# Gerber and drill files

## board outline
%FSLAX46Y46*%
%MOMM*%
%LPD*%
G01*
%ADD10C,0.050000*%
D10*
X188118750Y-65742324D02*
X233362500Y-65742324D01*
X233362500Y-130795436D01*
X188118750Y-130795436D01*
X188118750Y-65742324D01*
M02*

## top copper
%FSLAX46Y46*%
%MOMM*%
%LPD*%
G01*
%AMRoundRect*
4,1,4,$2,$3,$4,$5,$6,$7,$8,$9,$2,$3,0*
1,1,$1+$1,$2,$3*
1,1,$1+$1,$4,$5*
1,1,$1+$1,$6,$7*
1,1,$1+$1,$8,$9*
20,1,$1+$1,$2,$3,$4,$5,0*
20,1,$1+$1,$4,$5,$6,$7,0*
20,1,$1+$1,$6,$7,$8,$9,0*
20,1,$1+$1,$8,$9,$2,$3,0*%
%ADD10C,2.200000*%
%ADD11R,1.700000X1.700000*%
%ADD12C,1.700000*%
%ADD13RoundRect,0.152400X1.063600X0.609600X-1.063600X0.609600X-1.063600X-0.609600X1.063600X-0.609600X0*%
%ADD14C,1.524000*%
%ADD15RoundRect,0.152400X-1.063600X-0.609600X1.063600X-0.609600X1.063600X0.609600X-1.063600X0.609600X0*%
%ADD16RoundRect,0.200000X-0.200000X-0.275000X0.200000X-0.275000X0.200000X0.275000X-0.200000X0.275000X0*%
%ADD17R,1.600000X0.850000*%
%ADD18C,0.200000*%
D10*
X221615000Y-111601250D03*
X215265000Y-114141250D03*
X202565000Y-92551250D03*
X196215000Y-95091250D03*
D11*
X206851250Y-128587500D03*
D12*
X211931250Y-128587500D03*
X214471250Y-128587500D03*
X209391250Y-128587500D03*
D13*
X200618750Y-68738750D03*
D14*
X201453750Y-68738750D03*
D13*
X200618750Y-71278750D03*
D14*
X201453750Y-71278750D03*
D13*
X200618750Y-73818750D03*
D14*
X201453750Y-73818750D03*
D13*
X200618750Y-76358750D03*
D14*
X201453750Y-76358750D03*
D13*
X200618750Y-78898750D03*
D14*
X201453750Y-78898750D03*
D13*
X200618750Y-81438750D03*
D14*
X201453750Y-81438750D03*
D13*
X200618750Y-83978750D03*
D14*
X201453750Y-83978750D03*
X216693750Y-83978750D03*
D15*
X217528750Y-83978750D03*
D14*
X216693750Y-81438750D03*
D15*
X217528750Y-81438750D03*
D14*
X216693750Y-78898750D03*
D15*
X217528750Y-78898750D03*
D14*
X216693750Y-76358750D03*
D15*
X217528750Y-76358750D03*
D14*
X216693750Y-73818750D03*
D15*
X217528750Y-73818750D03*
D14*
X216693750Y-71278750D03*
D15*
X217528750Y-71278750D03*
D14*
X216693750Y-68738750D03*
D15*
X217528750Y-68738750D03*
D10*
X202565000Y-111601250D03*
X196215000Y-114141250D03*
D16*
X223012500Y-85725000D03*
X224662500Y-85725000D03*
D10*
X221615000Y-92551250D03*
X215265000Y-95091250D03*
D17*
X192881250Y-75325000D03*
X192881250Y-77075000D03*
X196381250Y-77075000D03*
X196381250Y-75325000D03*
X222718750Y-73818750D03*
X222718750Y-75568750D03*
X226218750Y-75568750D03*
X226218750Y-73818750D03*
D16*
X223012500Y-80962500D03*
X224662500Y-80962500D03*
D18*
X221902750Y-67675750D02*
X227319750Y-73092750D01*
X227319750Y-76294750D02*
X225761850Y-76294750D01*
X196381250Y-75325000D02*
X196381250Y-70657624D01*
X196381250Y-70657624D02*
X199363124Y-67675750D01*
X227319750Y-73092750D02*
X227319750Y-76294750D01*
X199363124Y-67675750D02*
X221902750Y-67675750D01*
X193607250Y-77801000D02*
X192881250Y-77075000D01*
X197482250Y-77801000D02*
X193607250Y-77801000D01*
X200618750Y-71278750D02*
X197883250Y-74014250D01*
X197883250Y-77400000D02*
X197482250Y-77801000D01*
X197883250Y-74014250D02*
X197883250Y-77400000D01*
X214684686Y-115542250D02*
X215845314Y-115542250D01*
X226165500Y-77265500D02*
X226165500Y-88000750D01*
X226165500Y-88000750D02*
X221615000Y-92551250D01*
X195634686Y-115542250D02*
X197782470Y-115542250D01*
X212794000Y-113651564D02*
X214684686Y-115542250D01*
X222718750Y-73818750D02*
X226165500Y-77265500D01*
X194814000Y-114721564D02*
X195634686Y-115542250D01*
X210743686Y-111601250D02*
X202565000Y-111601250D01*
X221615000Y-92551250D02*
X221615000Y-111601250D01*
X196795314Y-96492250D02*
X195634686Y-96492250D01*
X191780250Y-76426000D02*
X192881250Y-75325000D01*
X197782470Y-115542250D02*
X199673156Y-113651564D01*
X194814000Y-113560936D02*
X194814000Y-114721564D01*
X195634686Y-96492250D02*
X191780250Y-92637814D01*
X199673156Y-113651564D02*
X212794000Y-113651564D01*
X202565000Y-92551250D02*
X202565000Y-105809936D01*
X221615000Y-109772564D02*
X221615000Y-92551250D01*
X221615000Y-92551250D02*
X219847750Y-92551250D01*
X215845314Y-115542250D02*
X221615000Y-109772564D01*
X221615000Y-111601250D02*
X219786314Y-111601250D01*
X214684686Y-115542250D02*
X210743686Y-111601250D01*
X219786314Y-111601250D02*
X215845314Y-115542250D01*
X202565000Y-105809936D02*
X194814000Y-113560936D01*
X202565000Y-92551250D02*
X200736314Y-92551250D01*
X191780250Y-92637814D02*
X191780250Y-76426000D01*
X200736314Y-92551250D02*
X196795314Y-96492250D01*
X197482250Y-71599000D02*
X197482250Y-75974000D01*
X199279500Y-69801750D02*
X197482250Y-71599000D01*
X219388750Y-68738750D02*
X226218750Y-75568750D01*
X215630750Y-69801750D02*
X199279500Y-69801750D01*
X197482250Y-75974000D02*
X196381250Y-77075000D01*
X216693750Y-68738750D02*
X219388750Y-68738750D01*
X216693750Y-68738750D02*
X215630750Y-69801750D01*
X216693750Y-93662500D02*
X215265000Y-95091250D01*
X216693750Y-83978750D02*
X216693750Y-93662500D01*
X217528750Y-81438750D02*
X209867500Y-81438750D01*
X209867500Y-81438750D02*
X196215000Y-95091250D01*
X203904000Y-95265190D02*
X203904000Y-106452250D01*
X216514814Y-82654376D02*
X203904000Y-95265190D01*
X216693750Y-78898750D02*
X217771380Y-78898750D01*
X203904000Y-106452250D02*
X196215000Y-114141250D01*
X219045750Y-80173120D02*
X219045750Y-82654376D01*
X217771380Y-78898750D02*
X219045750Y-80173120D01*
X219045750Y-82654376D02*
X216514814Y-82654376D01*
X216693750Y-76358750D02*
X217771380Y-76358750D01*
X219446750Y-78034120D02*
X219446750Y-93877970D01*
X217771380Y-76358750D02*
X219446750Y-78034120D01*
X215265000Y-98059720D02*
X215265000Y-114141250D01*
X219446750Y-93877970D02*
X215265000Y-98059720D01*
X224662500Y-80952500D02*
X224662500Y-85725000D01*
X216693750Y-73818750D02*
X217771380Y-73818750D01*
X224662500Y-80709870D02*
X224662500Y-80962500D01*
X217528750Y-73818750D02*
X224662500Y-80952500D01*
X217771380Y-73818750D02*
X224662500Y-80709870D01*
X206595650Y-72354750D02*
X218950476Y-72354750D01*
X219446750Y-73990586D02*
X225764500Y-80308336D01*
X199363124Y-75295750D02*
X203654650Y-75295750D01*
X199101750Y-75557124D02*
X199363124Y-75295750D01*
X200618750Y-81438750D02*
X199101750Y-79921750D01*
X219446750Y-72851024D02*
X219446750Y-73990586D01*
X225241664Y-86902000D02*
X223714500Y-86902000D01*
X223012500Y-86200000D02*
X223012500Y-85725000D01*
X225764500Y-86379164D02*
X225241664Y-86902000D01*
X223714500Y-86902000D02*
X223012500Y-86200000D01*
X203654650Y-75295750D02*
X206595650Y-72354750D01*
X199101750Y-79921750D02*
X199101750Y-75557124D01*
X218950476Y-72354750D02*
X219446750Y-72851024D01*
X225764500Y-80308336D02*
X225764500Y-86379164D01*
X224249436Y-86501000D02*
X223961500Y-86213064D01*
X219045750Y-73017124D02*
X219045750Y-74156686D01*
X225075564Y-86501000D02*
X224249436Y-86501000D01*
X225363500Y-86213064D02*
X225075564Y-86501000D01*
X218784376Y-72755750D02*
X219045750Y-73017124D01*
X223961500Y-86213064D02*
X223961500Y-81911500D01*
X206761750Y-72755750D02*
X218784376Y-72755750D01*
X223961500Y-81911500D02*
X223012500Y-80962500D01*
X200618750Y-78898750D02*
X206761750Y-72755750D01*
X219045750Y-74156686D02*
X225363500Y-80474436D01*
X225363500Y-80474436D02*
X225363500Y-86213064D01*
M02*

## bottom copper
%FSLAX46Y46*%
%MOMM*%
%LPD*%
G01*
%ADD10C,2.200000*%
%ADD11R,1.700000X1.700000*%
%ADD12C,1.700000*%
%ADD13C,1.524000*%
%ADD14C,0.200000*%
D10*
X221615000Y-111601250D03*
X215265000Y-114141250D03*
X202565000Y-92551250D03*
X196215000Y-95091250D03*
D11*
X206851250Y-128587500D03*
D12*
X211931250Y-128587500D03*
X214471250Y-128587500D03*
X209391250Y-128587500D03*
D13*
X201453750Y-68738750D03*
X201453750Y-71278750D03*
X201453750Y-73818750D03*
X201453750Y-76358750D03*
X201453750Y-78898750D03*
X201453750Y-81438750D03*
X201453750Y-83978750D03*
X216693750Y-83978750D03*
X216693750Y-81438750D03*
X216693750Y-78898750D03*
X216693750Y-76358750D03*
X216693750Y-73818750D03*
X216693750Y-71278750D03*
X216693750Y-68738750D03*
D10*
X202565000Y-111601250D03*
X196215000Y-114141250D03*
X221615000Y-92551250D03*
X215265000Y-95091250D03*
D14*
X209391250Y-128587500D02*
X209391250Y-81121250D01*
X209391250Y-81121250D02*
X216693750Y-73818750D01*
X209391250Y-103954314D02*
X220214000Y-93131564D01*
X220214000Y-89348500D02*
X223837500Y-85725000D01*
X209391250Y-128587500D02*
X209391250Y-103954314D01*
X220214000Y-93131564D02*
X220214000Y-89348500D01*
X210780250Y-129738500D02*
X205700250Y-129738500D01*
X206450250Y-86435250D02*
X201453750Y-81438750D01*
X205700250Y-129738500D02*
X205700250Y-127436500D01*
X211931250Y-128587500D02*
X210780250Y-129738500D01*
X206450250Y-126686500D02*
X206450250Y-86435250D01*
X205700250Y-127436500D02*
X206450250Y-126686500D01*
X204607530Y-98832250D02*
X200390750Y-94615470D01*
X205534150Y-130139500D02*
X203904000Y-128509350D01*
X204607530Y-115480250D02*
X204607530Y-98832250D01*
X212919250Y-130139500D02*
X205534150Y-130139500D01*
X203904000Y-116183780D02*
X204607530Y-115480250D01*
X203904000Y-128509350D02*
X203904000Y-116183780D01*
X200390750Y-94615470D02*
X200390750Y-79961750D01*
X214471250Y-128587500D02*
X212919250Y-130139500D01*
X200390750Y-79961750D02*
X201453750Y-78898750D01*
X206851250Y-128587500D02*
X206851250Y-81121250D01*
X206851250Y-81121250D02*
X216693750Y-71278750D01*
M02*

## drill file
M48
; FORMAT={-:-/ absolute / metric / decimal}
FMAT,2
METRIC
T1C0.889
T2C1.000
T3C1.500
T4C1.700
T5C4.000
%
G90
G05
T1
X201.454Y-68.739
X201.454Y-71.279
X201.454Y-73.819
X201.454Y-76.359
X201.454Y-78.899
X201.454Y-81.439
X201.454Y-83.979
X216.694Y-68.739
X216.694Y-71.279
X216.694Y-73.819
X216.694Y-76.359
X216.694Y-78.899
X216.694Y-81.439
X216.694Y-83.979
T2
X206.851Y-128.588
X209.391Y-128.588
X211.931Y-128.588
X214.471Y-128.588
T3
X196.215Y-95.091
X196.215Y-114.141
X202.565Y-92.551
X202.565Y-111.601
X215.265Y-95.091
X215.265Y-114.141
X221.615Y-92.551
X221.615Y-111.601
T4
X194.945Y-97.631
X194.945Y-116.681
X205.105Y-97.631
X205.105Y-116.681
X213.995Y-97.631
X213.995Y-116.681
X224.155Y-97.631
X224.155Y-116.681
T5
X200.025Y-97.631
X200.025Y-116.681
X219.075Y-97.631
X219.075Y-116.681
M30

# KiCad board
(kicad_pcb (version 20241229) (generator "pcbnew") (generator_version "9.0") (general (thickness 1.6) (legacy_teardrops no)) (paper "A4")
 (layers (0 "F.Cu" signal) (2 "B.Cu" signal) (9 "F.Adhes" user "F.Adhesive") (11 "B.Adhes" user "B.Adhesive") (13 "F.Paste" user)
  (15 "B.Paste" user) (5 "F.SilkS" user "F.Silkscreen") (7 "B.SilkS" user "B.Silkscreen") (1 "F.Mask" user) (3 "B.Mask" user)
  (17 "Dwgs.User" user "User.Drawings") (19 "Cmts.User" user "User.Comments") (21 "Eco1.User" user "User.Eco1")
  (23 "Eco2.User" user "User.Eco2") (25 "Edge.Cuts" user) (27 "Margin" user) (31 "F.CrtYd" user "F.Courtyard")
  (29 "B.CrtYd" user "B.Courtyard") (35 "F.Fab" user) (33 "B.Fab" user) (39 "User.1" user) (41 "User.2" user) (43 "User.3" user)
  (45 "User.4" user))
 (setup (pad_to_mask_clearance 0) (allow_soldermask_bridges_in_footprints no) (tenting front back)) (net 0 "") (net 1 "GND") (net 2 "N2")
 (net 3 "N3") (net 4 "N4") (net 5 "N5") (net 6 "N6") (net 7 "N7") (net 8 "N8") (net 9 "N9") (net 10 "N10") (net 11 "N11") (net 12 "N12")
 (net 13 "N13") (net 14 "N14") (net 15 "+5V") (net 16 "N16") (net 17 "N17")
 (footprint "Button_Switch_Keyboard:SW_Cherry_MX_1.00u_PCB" (layer "F.Cu") (at 221.615 111.60125)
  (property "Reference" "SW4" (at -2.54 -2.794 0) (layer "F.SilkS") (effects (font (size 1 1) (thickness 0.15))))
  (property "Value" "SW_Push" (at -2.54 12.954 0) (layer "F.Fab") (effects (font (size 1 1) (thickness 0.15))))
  (pad "" np_thru_hole circle (at -7.62 5.08) (size 1.7 1.7) (drill 1.7) (layers "*.Cu" "*.Mask"))
  (pad "" np_thru_hole circle (at -2.54 5.08) (size 4 4) (drill 4) (layers "*.Cu" "*.Mask"))
  (pad "" np_thru_hole circle (at 2.54 5.08) (size 1.7 1.7) (drill 1.7) (layers "*.Cu" "*.Mask"))
  (pad "1" thru_hole circle (at 0 0) (size 2.2 2.2) (drill 1.5) (layers "*.Cu" "*.Mask") (remove_unused_layers no) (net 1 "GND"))
  (pad "2" thru_hole circle (at -6.35 2.54) (size 2.2 2.2) (drill 1.5) (layers "*.Cu" "*.Mask") (remove_unused_layers no) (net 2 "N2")))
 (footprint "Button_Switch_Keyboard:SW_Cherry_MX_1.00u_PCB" (layer "F.Cu") (at 202.565 92.55125)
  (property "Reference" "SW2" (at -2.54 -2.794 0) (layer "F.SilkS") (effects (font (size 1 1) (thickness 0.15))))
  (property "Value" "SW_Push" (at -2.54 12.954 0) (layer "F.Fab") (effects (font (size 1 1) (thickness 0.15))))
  (pad "" np_thru_hole circle (at -7.62 5.08) (size 1.7 1.7) (drill 1.7) (layers "*.Cu" "*.Mask"))
  (pad "" np_thru_hole circle (at -2.54 5.08) (size 4 4) (drill 4) (layers "*.Cu" "*.Mask"))
  (pad "" np_thru_hole circle (at 2.54 5.08) (size 1.7 1.7) (drill 1.7) (layers "*.Cu" "*.Mask"))
  (pad "1" thru_hole circle (at 0 0) (size 2.2 2.2) (drill 1.5) (layers "*.Cu" "*.Mask") (remove_unused_layers no) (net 1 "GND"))
  (pad "2" thru_hole circle (at -6.35 2.54) (size 2.2 2.2) (drill 1.5) (layers "*.Cu" "*.Mask") (remove_unused_layers no) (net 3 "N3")))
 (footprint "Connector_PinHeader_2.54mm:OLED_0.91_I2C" (layer "F.Cu") (at 206.85125 128.5875 90)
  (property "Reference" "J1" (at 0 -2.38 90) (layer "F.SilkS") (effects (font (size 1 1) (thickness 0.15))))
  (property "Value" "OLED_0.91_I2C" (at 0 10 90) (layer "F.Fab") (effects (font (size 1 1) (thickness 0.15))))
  (pad "GND" thru_hole rect (at 0 0 90) (size 1.7 1.7) (drill 1) (layers "*.Cu" "*.Mask") (remove_unused_layers no) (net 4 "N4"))
  (pad "SCL" thru_hole circle (at 0 5.08 90) (size 1.7 1.7) (drill 1) (layers "*.Cu" "*.Mask") (remove_unused_layers no) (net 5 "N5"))
  (pad "SDA" thru_hole circle (at 0 7.62 90) (size 1.7 1.7) (drill 1) (layers "*.Cu" "*.Mask") (remove_unused_layers no) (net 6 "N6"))
  (pad "VCC" thru_hole circle (at 0 2.54 90) (size 1.7 1.7) (drill 1) (layers "*.Cu" "*.Mask") (remove_unused_layers no) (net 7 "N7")))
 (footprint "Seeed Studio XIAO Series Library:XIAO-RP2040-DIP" (layer "F.Cu") (at 209.07375 76.35875)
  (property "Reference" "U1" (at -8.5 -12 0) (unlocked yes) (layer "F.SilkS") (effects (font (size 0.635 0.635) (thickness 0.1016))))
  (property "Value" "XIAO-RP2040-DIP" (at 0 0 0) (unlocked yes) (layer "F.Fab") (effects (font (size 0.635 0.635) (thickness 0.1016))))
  (pad "1" smd roundrect (at -8.455 -7.62 180) (size 2.432 1.524) (layers "F.Cu" "F.Mask") (roundrect_rratio 0.1) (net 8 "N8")
   (thermal_bridge_angle 45))
  (pad "1" thru_hole circle (at -7.62 -7.62 180) (size 1.524 1.524) (drill 0.889) (layers "*.Cu" "*.Mask") (remove_unused_layers no)
   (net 8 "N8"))
  (pad "2" smd roundrect (at -8.455 -5.08 180) (size 2.432 1.524) (layers "F.Cu" "F.Mask") (roundrect_rratio 0.1) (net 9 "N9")
   (thermal_bridge_angle 45))
  (pad "2" thru_hole circle (at -7.62 -5.08 180) (size 1.524 1.524) (drill 0.889) (layers "*.Cu" "*.Mask") (remove_unused_layers no)
   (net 9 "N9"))
  (pad "3" smd roundrect (at -8.455 -2.54 180) (size 2.432 1.524) (layers "F.Cu" "F.Mask") (roundrect_rratio 0.1) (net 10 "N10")
   (thermal_bridge_angle 45))
  (pad "3" thru_hole circle (at -7.62 -2.54 180) (size 1.524 1.524) (drill 0.889) (layers "*.Cu" "*.Mask") (remove_unused_layers no)
   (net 10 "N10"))
  (pad "4" smd roundrect (at -8.455 0 180) (size 2.432 1.524) (layers "F.Cu" "F.Mask") (roundrect_rratio 0.1) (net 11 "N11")
   (thermal_bridge_angle 45))
  (pad "4" thru_hole circle (at -7.62 0 180) (size 1.524 1.524) (drill 0.889) (layers "*.Cu" "*.Mask") (remove_unused_layers no)
   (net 11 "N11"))
  (pad "5" smd roundrect (at -8.455 2.54 180) (size 2.432 1.524) (layers "F.Cu" "F.Mask") (roundrect_rratio 0.1) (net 6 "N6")
   (thermal_bridge_angle 45))
  (pad "5" thru_hole circle (at -7.62 2.54 180) (size 1.524 1.524) (drill 0.889) (layers "*.Cu" "*.Mask") (remove_unused_layers no)
   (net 6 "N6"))
  (pad "6" smd roundrect (at -8.455 5.08 180) (size 2.432 1.524) (layers "F.Cu" "F.Mask") (roundrect_rratio 0.1) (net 5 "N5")
   (thermal_bridge_angle 45))
  (pad "6" thru_hole circle (at -7.62 5.08 180) (size 1.524 1.524) (drill 0.889) (layers "*.Cu" "*.Mask") (remove_unused_layers no)
   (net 5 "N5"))
  (pad "7" smd roundrect (at -8.455 7.62 180) (size 2.432 1.524) (layers "F.Cu" "F.Mask") (roundrect_rratio 0.1) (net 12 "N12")
   (thermal_bridge_angle 45))
  (pad "7" thru_hole circle (at -7.62 7.62 180) (size 1.524 1.524) (drill 0.889) (layers "*.Cu" "*.Mask") (remove_unused_layers no)
   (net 12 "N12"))
  (pad "8" thru_hole circle (at 7.62 7.62) (size 1.524 1.524) (drill 0.889) (layers "*.Cu" "*.Mask") (remove_unused_layers no)
   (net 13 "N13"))
  (pad "8" smd roundrect (at 8.455 7.62) (size 2.432 1.524) (layers "F.Cu" "F.Mask") (roundrect_rratio 0.1) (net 13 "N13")
   (thermal_bridge_angle 45))
  (pad "9" thru_hole circle (at 7.62 5.08) (size 1.524 1.524) (drill 0.889) (layers "*.Cu" "*.Mask") (remove_unused_layers no) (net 3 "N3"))
  (pad "9" smd roundrect (at 8.455 5.08) (size 2.432 1.524) (layers "F.Cu" "F.Mask") (roundrect_rratio 0.1) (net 3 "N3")
   (thermal_bridge_angle 45))
  (pad "10" thru_hole circle (at 7.62 2.54) (size 1.524 1.524) (drill 0.889) (layers "*.Cu" "*.Mask") (remove_unused_layers no)
   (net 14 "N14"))
  (pad "10" smd roundrect (at 8.455 2.54) (size 2.432 1.524) (layers "F.Cu" "F.Mask") (roundrect_rratio 0.1) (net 14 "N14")
   (thermal_bridge_angle 45))
  (pad "11" thru_hole circle (at 7.62 0) (size 1.524 1.524) (drill 0.889) (layers "*.Cu" "*.Mask") (remove_unused_layers no) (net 2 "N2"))
  (pad "11" smd roundrect (at 8.455 0) (size 2.432 1.524) (layers "F.Cu" "F.Mask") (roundrect_rratio 0.1) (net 2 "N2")
   (thermal_bridge_angle 45))
  (pad "12" thru_hole circle (at 7.62 -2.54) (size 1.524 1.524) (drill 0.889) (layers "*.Cu" "*.Mask") (remove_unused_layers no)
   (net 7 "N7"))
  (pad "12" smd roundrect (at 8.455 -2.54) (size 2.432 1.524) (layers "F.Cu" "F.Mask") (roundrect_rratio 0.1) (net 7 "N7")
   (thermal_bridge_angle 45))
  (pad "13" thru_hole circle (at 7.62 -5.08) (size 1.524 1.524) (drill 0.889) (layers "*.Cu" "*.Mask") (remove_unused_layers no)
   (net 4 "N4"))
  (pad "13" smd roundrect (at 8.455 -5.08) (size 2.432 1.524) (layers "F.Cu" "F.Mask") (roundrect_rratio 0.1) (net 4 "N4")
   (thermal_bridge_angle 45))
  (pad "14" thru_hole circle (at 7.62 -7.62) (size 1.524 1.524) (drill 0.889) (layers "*.Cu" "*.Mask") (remove_unused_layers no)
   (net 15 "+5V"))
  (pad "14" smd roundrect (at 8.455 -7.62) (size 2.432 1.524) (layers "F.Cu" "F.Mask") (roundrect_rratio 0.1) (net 15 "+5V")
   (thermal_bridge_angle 45)))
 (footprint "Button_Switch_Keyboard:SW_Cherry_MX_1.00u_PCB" (layer "F.Cu") (at 202.565 111.60125)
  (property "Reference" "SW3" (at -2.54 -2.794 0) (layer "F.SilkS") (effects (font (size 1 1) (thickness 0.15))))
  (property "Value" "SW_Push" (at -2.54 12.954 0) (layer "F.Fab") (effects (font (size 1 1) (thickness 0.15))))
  (pad "" np_thru_hole circle (at -7.62 5.08) (size 1.7 1.7) (drill 1.7) (layers "*.Cu" "*.Mask"))
  (pad "" np_thru_hole circle (at -2.54 5.08) (size 4 4) (drill 4) (layers "*.Cu" "*.Mask"))
  (pad "" np_thru_hole circle (at 2.54 5.08) (size 1.7 1.7) (drill 1.7) (layers "*.Cu" "*.Mask"))
  (pad "1" thru_hole circle (at 0 0) (size 2.2 2.2) (drill 1.5) (layers "*.Cu" "*.Mask") (remove_unused_layers no) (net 1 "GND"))
  (pad "2" thru_hole circle (at -6.35 2.54) (size 2.2 2.2) (drill 1.5) (layers "*.Cu" "*.Mask") (remove_unused_layers no) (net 14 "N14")))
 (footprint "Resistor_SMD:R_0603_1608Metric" (layer "F.Cu") (at 223.8375 85.725)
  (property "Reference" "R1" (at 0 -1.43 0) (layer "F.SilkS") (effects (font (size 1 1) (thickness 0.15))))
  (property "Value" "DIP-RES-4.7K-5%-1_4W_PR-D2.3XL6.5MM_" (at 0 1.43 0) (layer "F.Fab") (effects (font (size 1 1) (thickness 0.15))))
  (pad "1" smd roundrect (at -0.825 0) (size 0.8 0.95) (layers "F.Cu" "F.Mask" "F.Paste") (roundrect_rratio 0.25) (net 5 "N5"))
  (pad "2" smd roundrect (at 0.825 0) (size 0.8 0.95) (layers "F.Cu" "F.Mask" "F.Paste") (roundrect_rratio 0.25) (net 7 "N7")))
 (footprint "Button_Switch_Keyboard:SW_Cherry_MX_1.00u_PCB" (layer "F.Cu") (at 221.615 92.55125)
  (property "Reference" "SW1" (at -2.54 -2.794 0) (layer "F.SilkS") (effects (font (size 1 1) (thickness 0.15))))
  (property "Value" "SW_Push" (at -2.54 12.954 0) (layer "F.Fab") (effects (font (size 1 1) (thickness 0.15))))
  (pad "" np_thru_hole circle (at -7.62 5.08) (size 1.7 1.7) (drill 1.7) (layers "*.Cu" "*.Mask"))
  (pad "" np_thru_hole circle (at -2.54 5.08) (size 4 4) (drill 4) (layers "*.Cu" "*.Mask"))
  (pad "" np_thru_hole circle (at 2.54 5.08) (size 1.7 1.7) (drill 1.7) (layers "*.Cu" "*.Mask"))
  (pad "1" thru_hole circle (at 0 0) (size 2.2 2.2) (drill 1.5) (layers "*.Cu" "*.Mask") (remove_unused_layers no) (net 1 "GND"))
  (pad "2" thru_hole circle (at -6.35 2.54) (size 2.2 2.2) (drill 1.5) (layers "*.Cu" "*.Mask") (remove_unused_layers no) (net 13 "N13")))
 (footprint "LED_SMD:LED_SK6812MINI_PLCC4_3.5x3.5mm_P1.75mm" (layer "F.Cu") (at 194.63125 76.2)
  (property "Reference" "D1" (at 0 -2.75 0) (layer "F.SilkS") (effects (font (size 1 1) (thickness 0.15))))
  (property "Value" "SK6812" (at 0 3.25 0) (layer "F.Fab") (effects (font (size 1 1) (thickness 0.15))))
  (pad "1" smd rect (at -1.75 -0.875) (size 1.6 0.85) (layers "F.Cu" "F.Mask" "F.Paste") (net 1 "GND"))
  (pad "2" smd rect (at -1.75 0.875) (size 1.6 0.85) (layers "F.Cu" "F.Mask" "F.Paste") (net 9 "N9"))
  (pad "3" smd rect (at 1.75 0.875) (size 1.6 0.85) (layers "F.Cu" "F.Mask" "F.Paste") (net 15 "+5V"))
  (pad "4" smd rect (at 1.75 -0.875) (size 1.6 0.85) (layers "F.Cu" "F.Mask" "F.Paste") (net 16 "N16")))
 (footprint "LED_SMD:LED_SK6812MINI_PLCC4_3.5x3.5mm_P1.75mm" (layer "F.Cu") (at 224.46875 74.69375)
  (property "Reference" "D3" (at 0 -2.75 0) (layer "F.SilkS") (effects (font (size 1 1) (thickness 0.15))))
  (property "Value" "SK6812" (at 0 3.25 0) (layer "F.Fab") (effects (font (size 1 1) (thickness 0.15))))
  (pad "1" smd rect (at -1.75 -0.875) (size 1.6 0.85) (layers "F.Cu" "F.Mask" "F.Paste") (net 1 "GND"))
  (pad "2" smd rect (at -1.75 0.875) (size 1.6 0.85) (layers "F.Cu" "F.Mask" "F.Paste") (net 16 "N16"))
  (pad "3" smd rect (at 1.75 0.875) (size 1.6 0.85) (layers "F.Cu" "F.Mask" "F.Paste") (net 15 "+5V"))
  (pad "4" smd rect (at 1.75 -0.875) (size 1.6 0.85) (layers "F.Cu" "F.Mask" "F.Paste") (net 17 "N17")))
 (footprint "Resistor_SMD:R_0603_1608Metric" (layer "F.Cu") (at 223.8375 80.9625)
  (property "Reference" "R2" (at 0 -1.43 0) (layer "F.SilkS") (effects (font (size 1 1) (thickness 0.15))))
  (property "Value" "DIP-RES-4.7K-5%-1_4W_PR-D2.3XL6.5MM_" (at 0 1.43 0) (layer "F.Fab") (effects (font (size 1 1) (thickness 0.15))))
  (pad "1" smd roundrect (at -0.825 0) (size 0.8 0.95) (layers "F.Cu" "F.Mask" "F.Paste") (roundrect_rratio 0.25) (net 6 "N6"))
  (pad "2" smd roundrect (at 0.825 0) (size 0.8 0.95) (layers "F.Cu" "F.Mask" "F.Paste") (roundrect_rratio 0.25) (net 7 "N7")))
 (gr_rect (start 188.11875 65.742324) (end 233.3625 130.795436) (stroke (width 0.05) (type default)) (fill no) (layer "Edge.Cuts"))
 (segment (start 221.90275 67.67575) (end 227.31975 73.09275) (width 0.2) (layer "F.Cu") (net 16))
 (segment (start 227.31975 76.29475) (end 225.76185 76.29475) (width 0.2) (layer "F.Cu") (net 16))
 (segment (start 196.38125 75.325) (end 196.38125 70.657624) (width 0.2) (layer "F.Cu") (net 16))
 (segment (start 196.38125 70.657624) (end 199.363124 67.67575) (width 0.2) (layer "F.Cu") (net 16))
 (segment (start 227.31975 73.09275) (end 227.31975 76.29475) (width 0.2) (layer "F.Cu") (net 16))
 (segment (start 199.363124 67.67575) (end 221.90275 67.67575) (width 0.2) (layer "F.Cu") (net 16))
 (segment (start 193.60725 77.801) (end 192.88125 77.075) (width 0.2) (layer "F.Cu") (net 9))
 (segment (start 197.48225 77.801) (end 193.60725 77.801) (width 0.2) (layer "F.Cu") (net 9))
 (segment (start 200.61875 71.27875) (end 197.88325 74.01425) (width 0.2) (layer "F.Cu") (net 9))
 (segment (start 197.88325 77.4) (end 197.48225 77.801) (width 0.2) (layer "F.Cu") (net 9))
 (segment (start 197.88325 74.01425) (end 197.88325 77.4) (width 0.2) (layer "F.Cu") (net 9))
 (segment (start 214.684686 115.54225) (end 215.845314 115.54225) (width 0.2) (layer "F.Cu") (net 1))
 (segment (start 226.1655 77.2655) (end 226.1655 88.00075) (width 0.2) (layer "F.Cu") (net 1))
 (segment (start 226.1655 88.00075) (end 221.615 92.55125) (width 0.2) (layer "F.Cu") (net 1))
 (segment (start 195.634686 115.54225) (end 197.78247 115.54225) (width 0.2) (layer "F.Cu") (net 1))
 (segment (start 212.794 113.651564) (end 214.684686 115.54225) (width 0.2) (layer "F.Cu") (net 1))
 (segment (start 222.71875 73.81875) (end 226.1655 77.2655) (width 0.2) (layer "F.Cu") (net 1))
 (segment (start 194.814 114.721564) (end 195.634686 115.54225) (width 0.2) (layer "F.Cu") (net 1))
 (segment (start 210.743686 111.60125) (end 202.565 111.60125) (width 0.2) (layer "F.Cu") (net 1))
 (segment (start 221.615 92.55125) (end 221.615 111.60125) (width 0.2) (layer "F.Cu") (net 1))
 (segment (start 196.795314 96.49225) (end 195.634686 96.49225) (width 0.2) (layer "F.Cu") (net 1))
 (segment (start 191.78025 76.426) (end 192.88125 75.325) (width 0.2) (layer "F.Cu") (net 1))
 (segment (start 197.78247 115.54225) (end 199.673156 113.651564) (width 0.2) (layer "F.Cu") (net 1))
 (segment (start 194.814 113.560936) (end 194.814 114.721564) (width 0.2) (layer "F.Cu") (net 1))
 (segment (start 195.634686 96.49225) (end 191.78025 92.637814) (width 0.2) (layer "F.Cu") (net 1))
 (segment (start 199.673156 113.651564) (end 212.794 113.651564) (width 0.2) (layer "F.Cu") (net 1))
 (segment (start 202.565 92.55125) (end 202.565 105.809936) (width 0.2) (layer "F.Cu") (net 1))
 (segment (start 221.615 109.772564) (end 221.615 92.55125) (width 0.2) (layer "F.Cu") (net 1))
 (segment (start 221.615 92.55125) (end 219.84775 92.55125) (width 0.2) (layer "F.Cu") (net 1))
 (segment (start 215.845314 115.54225) (end 221.615 109.772564) (width 0.2) (layer "F.Cu") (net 1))
 (segment (start 221.615 111.60125) (end 219.786314 111.60125) (width 0.2) (layer "F.Cu") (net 1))
 (segment (start 214.684686 115.54225) (end 210.743686 111.60125) (width 0.2) (layer "F.Cu") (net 1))
 (segment (start 219.786314 111.60125) (end 215.845314 115.54225) (width 0.2) (layer "F.Cu") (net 1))
 (segment (start 202.565 105.809936) (end 194.814 113.560936) (width 0.2) (layer "F.Cu") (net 1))
 (segment (start 202.565 92.55125) (end 200.736314 92.55125) (width 0.2) (layer "F.Cu") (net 1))
 (segment (start 191.78025 92.637814) (end 191.78025 76.426) (width 0.2) (layer "F.Cu") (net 1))
 (segment (start 200.736314 92.55125) (end 196.795314 96.49225) (width 0.2) (layer "F.Cu") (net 1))
 (segment (start 197.48225 71.599) (end 197.48225 75.974) (width 0.2) (layer "F.Cu") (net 15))
 (segment (start 199.2795 69.80175) (end 197.48225 71.599) (width 0.2) (layer "F.Cu") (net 15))
 (segment (start 219.38875 68.73875) (end 226.21875 75.56875) (width 0.2) (layer "F.Cu") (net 15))
 (segment (start 215.63075 69.80175) (end 199.2795 69.80175) (width 0.2) (layer "F.Cu") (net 15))
 (segment (start 197.48225 75.974) (end 196.38125 77.075) (width 0.2) (layer "F.Cu") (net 15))
 (segment (start 216.69375 68.73875) (end 219.38875 68.73875) (width 0.2) (layer "F.Cu") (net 15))
 (segment (start 216.69375 68.73875) (end 215.63075 69.80175) (width 0.2) (layer "F.Cu") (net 15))
 (segment (start 216.69375 93.6625) (end 215.265 95.09125) (width 0.2) (layer "F.Cu") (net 13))
 (segment (start 216.69375 83.97875) (end 216.69375 93.6625) (width 0.2) (layer "F.Cu") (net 13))
 (segment (start 217.52875 81.43875) (end 209.8675 81.43875) (width 0.2) (layer "F.Cu") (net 3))
 (segment (start 209.8675 81.43875) (end 196.215 95.09125) (width 0.2) (layer "F.Cu") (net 3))
 (segment (start 203.904 95.26519) (end 203.904 106.45225) (width 0.2) (layer "F.Cu") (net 14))
 (segment (start 216.514814 82.654376) (end 203.904 95.26519) (width 0.2) (layer "F.Cu") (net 14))
 (segment (start 216.69375 78.89875) (end 217.77138 78.89875) (width 0.2) (layer "F.Cu") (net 14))
 (segment (start 203.904 106.45225) (end 196.215 114.14125) (width 0.2) (layer "F.Cu") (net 14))
 (segment (start 219.04575 80.17312) (end 219.04575 82.654376) (width 0.2) (layer "F.Cu") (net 14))
 (segment (start 217.77138 78.89875) (end 219.04575 80.17312) (width 0.2) (layer "F.Cu") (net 14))
 (segment (start 219.04575 82.654376) (end 216.514814 82.654376) (width 0.2) (layer "F.Cu") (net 14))
 (segment (start 216.69375 76.35875) (end 217.77138 76.35875) (width 0.2) (layer "F.Cu") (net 2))
 (segment (start 219.44675 78.03412) (end 219.44675 93.87797) (width 0.2) (layer "F.Cu") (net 2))
 (segment (start 217.77138 76.35875) (end 219.44675 78.03412) (width 0.2) (layer "F.Cu") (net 2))
 (segment (start 215.265 98.05972) (end 215.265 114.14125) (width 0.2) (layer "F.Cu") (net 2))
 (segment (start 219.44675 93.87797) (end 215.265 98.05972) (width 0.2) (layer "F.Cu") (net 2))
 (segment (start 224.6625 80.9525) (end 224.6625 85.725) (width 0.2) (layer "F.Cu") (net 7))
 (segment (start 216.69375 73.81875) (end 217.77138 73.81875) (width 0.2) (layer "F.Cu") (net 7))
 (segment (start 224.6625 80.70987) (end 224.6625 80.9625) (width 0.2) (layer "F.Cu") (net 7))
 (segment (start 217.52875 73.81875) (end 224.6625 80.9525) (width 0.2) (layer "F.Cu") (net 7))
 (segment (start 217.77138 73.81875) (end 224.6625 80.70987) (width 0.2) (layer "F.Cu") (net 7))
 (segment (start 209.39125 128.5875) (end 209.39125 81.12125) (width 0.2) (layer "B.Cu") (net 7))
 (segment (start 209.39125 81.12125) (end 216.69375 73.81875) (width 0.2) (layer "B.Cu") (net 7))
 (segment (start 209.39125 103.954314) (end 220.214 93.131564) (width 0.2) (layer "B.Cu") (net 7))
 (segment (start 220.214 89.3485) (end 223.8375 85.725) (width 0.2) (layer "B.Cu") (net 7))
 (segment (start 209.39125 128.5875) (end 209.39125 103.954314) (width 0.2) (layer "B.Cu") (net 7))
 (segment (start 220.214 93.131564) (end 220.214 89.3485) (width 0.2) (layer "B.Cu") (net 7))
 (segment (start 206.59565 72.35475) (end 218.950476 72.35475) (width 0.2) (layer "F.Cu") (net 5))
 (segment (start 219.44675 73.990586) (end 225.7645 80.308336) (width 0.2) (layer "F.Cu") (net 5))
 (segment (start 199.363124 75.29575) (end 203.65465 75.29575) (width 0.2) (layer "F.Cu") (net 5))
 (segment (start 199.10175 75.557124) (end 199.363124 75.29575) (width 0.2) (layer "F.Cu") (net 5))
 (segment (start 200.61875 81.43875) (end 199.10175 79.92175) (width 0.2) (layer "F.Cu") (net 5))
 (segment (start 219.44675 72.851024) (end 219.44675 73.990586) (width 0.2) (layer "F.Cu") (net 5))
 (segment (start 225.241664 86.902) (end 223.7145 86.902) (width 0.2) (layer "F.Cu") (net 5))
 (segment (start 223.0125 86.2) (end 223.0125 85.725) (width 0.2) (layer "F.Cu") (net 5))
 (segment (start 225.7645 86.379164) (end 225.241664 86.902) (width 0.2) (layer "F.Cu") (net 5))
 (segment (start 223.7145 86.902) (end 223.0125 86.2) (width 0.2) (layer "F.Cu") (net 5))
 (segment (start 203.65465 75.29575) (end 206.59565 72.35475) (width 0.2) (layer "F.Cu") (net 5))
 (segment (start 199.10175 79.92175) (end 199.10175 75.557124) (width 0.2) (layer "F.Cu") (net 5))
 (segment (start 218.950476 72.35475) (end 219.44675 72.851024) (width 0.2) (layer "F.Cu") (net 5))
 (segment (start 225.7645 80.308336) (end 225.7645 86.379164) (width 0.2) (layer "F.Cu") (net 5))
 (segment (start 210.78025 129.7385) (end 205.70025 129.7385) (width 0.2) (layer "B.Cu") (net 5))
 (segment (start 206.45025 86.43525) (end 201.45375 81.43875) (width 0.2) (layer "B.Cu") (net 5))
 (segment (start 205.70025 129.7385) (end 205.70025 127.4365) (width 0.2) (layer "B.Cu") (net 5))
 (segment (start 211.93125 128.5875) (end 210.78025 129.7385) (width 0.2) (layer "B.Cu") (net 5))
 (segment (start 206.45025 126.6865) (end 206.45025 86.43525) (width 0.2) (layer "B.Cu") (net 5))
 (segment (start 205.70025 127.4365) (end 206.45025 126.6865) (width 0.2) (layer "B.Cu") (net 5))
 (segment (start 224.249436 86.501) (end 223.9615 86.213064) (width 0.2) (layer "F.Cu") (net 6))
 (segment (start 219.04575 73.017124) (end 219.04575 74.156686) (width 0.2) (layer "F.Cu") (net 6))
 (segment (start 225.075564 86.501) (end 224.249436 86.501) (width 0.2) (layer "F.Cu") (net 6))
 (segment (start 225.3635 86.213064) (end 225.075564 86.501) (width 0.2) (layer "F.Cu") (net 6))
 (segment (start 218.784376 72.75575) (end 219.04575 73.017124) (width 0.2) (layer "F.Cu") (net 6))
 (segment (start 223.9615 86.213064) (end 223.9615 81.9115) (width 0.2) (layer "F.Cu") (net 6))
 (segment (start 206.76175 72.75575) (end 218.784376 72.75575) (width 0.2) (layer "F.Cu") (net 6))
 (segment (start 223.9615 81.9115) (end 223.0125 80.9625) (width 0.2) (layer "F.Cu") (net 6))
 (segment (start 200.61875 78.89875) (end 206.76175 72.75575) (width 0.2) (layer "F.Cu") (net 6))
 (segment (start 219.04575 74.156686) (end 225.3635 80.474436) (width 0.2) (layer "F.Cu") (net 6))
 (segment (start 225.3635 80.474436) (end 225.3635 86.213064) (width 0.2) (layer "F.Cu") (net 6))
 (segment (start 204.60753 98.83225) (end 200.39075 94.61547) (width 0.2) (layer "B.Cu") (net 6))
 (segment (start 205.53415 130.1395) (end 203.904 128.50935) (width 0.2) (layer "B.Cu") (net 6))
 (segment (start 204.60753 115.48025) (end 204.60753 98.83225) (width 0.2) (layer "B.Cu") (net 6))
 (segment (start 212.91925 130.1395) (end 205.53415 130.1395) (width 0.2) (layer "B.Cu") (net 6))
 (segment (start 203.904 116.18378) (end 204.60753 115.48025) (width 0.2) (layer "B.Cu") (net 6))
 (segment (start 203.904 128.50935) (end 203.904 116.18378) (width 0.2) (layer "B.Cu") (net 6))
 (segment (start 200.39075 94.61547) (end 200.39075 79.96175) (width 0.2) (layer "B.Cu") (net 6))
 (segment (start 214.47125 128.5875) (end 212.91925 130.1395) (width 0.2) (layer "B.Cu") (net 6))
 (segment (start 200.39075 79.96175) (end 201.45375 78.89875) (width 0.2) (layer "B.Cu") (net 6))
 (segment (start 206.85125 128.5875) (end 206.85125 81.12125) (width 0.2) (layer "B.Cu") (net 4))
 (segment (start 206.85125 81.12125) (end 216.69375 71.27875) (width 0.2) (layer "B.Cu") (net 4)))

